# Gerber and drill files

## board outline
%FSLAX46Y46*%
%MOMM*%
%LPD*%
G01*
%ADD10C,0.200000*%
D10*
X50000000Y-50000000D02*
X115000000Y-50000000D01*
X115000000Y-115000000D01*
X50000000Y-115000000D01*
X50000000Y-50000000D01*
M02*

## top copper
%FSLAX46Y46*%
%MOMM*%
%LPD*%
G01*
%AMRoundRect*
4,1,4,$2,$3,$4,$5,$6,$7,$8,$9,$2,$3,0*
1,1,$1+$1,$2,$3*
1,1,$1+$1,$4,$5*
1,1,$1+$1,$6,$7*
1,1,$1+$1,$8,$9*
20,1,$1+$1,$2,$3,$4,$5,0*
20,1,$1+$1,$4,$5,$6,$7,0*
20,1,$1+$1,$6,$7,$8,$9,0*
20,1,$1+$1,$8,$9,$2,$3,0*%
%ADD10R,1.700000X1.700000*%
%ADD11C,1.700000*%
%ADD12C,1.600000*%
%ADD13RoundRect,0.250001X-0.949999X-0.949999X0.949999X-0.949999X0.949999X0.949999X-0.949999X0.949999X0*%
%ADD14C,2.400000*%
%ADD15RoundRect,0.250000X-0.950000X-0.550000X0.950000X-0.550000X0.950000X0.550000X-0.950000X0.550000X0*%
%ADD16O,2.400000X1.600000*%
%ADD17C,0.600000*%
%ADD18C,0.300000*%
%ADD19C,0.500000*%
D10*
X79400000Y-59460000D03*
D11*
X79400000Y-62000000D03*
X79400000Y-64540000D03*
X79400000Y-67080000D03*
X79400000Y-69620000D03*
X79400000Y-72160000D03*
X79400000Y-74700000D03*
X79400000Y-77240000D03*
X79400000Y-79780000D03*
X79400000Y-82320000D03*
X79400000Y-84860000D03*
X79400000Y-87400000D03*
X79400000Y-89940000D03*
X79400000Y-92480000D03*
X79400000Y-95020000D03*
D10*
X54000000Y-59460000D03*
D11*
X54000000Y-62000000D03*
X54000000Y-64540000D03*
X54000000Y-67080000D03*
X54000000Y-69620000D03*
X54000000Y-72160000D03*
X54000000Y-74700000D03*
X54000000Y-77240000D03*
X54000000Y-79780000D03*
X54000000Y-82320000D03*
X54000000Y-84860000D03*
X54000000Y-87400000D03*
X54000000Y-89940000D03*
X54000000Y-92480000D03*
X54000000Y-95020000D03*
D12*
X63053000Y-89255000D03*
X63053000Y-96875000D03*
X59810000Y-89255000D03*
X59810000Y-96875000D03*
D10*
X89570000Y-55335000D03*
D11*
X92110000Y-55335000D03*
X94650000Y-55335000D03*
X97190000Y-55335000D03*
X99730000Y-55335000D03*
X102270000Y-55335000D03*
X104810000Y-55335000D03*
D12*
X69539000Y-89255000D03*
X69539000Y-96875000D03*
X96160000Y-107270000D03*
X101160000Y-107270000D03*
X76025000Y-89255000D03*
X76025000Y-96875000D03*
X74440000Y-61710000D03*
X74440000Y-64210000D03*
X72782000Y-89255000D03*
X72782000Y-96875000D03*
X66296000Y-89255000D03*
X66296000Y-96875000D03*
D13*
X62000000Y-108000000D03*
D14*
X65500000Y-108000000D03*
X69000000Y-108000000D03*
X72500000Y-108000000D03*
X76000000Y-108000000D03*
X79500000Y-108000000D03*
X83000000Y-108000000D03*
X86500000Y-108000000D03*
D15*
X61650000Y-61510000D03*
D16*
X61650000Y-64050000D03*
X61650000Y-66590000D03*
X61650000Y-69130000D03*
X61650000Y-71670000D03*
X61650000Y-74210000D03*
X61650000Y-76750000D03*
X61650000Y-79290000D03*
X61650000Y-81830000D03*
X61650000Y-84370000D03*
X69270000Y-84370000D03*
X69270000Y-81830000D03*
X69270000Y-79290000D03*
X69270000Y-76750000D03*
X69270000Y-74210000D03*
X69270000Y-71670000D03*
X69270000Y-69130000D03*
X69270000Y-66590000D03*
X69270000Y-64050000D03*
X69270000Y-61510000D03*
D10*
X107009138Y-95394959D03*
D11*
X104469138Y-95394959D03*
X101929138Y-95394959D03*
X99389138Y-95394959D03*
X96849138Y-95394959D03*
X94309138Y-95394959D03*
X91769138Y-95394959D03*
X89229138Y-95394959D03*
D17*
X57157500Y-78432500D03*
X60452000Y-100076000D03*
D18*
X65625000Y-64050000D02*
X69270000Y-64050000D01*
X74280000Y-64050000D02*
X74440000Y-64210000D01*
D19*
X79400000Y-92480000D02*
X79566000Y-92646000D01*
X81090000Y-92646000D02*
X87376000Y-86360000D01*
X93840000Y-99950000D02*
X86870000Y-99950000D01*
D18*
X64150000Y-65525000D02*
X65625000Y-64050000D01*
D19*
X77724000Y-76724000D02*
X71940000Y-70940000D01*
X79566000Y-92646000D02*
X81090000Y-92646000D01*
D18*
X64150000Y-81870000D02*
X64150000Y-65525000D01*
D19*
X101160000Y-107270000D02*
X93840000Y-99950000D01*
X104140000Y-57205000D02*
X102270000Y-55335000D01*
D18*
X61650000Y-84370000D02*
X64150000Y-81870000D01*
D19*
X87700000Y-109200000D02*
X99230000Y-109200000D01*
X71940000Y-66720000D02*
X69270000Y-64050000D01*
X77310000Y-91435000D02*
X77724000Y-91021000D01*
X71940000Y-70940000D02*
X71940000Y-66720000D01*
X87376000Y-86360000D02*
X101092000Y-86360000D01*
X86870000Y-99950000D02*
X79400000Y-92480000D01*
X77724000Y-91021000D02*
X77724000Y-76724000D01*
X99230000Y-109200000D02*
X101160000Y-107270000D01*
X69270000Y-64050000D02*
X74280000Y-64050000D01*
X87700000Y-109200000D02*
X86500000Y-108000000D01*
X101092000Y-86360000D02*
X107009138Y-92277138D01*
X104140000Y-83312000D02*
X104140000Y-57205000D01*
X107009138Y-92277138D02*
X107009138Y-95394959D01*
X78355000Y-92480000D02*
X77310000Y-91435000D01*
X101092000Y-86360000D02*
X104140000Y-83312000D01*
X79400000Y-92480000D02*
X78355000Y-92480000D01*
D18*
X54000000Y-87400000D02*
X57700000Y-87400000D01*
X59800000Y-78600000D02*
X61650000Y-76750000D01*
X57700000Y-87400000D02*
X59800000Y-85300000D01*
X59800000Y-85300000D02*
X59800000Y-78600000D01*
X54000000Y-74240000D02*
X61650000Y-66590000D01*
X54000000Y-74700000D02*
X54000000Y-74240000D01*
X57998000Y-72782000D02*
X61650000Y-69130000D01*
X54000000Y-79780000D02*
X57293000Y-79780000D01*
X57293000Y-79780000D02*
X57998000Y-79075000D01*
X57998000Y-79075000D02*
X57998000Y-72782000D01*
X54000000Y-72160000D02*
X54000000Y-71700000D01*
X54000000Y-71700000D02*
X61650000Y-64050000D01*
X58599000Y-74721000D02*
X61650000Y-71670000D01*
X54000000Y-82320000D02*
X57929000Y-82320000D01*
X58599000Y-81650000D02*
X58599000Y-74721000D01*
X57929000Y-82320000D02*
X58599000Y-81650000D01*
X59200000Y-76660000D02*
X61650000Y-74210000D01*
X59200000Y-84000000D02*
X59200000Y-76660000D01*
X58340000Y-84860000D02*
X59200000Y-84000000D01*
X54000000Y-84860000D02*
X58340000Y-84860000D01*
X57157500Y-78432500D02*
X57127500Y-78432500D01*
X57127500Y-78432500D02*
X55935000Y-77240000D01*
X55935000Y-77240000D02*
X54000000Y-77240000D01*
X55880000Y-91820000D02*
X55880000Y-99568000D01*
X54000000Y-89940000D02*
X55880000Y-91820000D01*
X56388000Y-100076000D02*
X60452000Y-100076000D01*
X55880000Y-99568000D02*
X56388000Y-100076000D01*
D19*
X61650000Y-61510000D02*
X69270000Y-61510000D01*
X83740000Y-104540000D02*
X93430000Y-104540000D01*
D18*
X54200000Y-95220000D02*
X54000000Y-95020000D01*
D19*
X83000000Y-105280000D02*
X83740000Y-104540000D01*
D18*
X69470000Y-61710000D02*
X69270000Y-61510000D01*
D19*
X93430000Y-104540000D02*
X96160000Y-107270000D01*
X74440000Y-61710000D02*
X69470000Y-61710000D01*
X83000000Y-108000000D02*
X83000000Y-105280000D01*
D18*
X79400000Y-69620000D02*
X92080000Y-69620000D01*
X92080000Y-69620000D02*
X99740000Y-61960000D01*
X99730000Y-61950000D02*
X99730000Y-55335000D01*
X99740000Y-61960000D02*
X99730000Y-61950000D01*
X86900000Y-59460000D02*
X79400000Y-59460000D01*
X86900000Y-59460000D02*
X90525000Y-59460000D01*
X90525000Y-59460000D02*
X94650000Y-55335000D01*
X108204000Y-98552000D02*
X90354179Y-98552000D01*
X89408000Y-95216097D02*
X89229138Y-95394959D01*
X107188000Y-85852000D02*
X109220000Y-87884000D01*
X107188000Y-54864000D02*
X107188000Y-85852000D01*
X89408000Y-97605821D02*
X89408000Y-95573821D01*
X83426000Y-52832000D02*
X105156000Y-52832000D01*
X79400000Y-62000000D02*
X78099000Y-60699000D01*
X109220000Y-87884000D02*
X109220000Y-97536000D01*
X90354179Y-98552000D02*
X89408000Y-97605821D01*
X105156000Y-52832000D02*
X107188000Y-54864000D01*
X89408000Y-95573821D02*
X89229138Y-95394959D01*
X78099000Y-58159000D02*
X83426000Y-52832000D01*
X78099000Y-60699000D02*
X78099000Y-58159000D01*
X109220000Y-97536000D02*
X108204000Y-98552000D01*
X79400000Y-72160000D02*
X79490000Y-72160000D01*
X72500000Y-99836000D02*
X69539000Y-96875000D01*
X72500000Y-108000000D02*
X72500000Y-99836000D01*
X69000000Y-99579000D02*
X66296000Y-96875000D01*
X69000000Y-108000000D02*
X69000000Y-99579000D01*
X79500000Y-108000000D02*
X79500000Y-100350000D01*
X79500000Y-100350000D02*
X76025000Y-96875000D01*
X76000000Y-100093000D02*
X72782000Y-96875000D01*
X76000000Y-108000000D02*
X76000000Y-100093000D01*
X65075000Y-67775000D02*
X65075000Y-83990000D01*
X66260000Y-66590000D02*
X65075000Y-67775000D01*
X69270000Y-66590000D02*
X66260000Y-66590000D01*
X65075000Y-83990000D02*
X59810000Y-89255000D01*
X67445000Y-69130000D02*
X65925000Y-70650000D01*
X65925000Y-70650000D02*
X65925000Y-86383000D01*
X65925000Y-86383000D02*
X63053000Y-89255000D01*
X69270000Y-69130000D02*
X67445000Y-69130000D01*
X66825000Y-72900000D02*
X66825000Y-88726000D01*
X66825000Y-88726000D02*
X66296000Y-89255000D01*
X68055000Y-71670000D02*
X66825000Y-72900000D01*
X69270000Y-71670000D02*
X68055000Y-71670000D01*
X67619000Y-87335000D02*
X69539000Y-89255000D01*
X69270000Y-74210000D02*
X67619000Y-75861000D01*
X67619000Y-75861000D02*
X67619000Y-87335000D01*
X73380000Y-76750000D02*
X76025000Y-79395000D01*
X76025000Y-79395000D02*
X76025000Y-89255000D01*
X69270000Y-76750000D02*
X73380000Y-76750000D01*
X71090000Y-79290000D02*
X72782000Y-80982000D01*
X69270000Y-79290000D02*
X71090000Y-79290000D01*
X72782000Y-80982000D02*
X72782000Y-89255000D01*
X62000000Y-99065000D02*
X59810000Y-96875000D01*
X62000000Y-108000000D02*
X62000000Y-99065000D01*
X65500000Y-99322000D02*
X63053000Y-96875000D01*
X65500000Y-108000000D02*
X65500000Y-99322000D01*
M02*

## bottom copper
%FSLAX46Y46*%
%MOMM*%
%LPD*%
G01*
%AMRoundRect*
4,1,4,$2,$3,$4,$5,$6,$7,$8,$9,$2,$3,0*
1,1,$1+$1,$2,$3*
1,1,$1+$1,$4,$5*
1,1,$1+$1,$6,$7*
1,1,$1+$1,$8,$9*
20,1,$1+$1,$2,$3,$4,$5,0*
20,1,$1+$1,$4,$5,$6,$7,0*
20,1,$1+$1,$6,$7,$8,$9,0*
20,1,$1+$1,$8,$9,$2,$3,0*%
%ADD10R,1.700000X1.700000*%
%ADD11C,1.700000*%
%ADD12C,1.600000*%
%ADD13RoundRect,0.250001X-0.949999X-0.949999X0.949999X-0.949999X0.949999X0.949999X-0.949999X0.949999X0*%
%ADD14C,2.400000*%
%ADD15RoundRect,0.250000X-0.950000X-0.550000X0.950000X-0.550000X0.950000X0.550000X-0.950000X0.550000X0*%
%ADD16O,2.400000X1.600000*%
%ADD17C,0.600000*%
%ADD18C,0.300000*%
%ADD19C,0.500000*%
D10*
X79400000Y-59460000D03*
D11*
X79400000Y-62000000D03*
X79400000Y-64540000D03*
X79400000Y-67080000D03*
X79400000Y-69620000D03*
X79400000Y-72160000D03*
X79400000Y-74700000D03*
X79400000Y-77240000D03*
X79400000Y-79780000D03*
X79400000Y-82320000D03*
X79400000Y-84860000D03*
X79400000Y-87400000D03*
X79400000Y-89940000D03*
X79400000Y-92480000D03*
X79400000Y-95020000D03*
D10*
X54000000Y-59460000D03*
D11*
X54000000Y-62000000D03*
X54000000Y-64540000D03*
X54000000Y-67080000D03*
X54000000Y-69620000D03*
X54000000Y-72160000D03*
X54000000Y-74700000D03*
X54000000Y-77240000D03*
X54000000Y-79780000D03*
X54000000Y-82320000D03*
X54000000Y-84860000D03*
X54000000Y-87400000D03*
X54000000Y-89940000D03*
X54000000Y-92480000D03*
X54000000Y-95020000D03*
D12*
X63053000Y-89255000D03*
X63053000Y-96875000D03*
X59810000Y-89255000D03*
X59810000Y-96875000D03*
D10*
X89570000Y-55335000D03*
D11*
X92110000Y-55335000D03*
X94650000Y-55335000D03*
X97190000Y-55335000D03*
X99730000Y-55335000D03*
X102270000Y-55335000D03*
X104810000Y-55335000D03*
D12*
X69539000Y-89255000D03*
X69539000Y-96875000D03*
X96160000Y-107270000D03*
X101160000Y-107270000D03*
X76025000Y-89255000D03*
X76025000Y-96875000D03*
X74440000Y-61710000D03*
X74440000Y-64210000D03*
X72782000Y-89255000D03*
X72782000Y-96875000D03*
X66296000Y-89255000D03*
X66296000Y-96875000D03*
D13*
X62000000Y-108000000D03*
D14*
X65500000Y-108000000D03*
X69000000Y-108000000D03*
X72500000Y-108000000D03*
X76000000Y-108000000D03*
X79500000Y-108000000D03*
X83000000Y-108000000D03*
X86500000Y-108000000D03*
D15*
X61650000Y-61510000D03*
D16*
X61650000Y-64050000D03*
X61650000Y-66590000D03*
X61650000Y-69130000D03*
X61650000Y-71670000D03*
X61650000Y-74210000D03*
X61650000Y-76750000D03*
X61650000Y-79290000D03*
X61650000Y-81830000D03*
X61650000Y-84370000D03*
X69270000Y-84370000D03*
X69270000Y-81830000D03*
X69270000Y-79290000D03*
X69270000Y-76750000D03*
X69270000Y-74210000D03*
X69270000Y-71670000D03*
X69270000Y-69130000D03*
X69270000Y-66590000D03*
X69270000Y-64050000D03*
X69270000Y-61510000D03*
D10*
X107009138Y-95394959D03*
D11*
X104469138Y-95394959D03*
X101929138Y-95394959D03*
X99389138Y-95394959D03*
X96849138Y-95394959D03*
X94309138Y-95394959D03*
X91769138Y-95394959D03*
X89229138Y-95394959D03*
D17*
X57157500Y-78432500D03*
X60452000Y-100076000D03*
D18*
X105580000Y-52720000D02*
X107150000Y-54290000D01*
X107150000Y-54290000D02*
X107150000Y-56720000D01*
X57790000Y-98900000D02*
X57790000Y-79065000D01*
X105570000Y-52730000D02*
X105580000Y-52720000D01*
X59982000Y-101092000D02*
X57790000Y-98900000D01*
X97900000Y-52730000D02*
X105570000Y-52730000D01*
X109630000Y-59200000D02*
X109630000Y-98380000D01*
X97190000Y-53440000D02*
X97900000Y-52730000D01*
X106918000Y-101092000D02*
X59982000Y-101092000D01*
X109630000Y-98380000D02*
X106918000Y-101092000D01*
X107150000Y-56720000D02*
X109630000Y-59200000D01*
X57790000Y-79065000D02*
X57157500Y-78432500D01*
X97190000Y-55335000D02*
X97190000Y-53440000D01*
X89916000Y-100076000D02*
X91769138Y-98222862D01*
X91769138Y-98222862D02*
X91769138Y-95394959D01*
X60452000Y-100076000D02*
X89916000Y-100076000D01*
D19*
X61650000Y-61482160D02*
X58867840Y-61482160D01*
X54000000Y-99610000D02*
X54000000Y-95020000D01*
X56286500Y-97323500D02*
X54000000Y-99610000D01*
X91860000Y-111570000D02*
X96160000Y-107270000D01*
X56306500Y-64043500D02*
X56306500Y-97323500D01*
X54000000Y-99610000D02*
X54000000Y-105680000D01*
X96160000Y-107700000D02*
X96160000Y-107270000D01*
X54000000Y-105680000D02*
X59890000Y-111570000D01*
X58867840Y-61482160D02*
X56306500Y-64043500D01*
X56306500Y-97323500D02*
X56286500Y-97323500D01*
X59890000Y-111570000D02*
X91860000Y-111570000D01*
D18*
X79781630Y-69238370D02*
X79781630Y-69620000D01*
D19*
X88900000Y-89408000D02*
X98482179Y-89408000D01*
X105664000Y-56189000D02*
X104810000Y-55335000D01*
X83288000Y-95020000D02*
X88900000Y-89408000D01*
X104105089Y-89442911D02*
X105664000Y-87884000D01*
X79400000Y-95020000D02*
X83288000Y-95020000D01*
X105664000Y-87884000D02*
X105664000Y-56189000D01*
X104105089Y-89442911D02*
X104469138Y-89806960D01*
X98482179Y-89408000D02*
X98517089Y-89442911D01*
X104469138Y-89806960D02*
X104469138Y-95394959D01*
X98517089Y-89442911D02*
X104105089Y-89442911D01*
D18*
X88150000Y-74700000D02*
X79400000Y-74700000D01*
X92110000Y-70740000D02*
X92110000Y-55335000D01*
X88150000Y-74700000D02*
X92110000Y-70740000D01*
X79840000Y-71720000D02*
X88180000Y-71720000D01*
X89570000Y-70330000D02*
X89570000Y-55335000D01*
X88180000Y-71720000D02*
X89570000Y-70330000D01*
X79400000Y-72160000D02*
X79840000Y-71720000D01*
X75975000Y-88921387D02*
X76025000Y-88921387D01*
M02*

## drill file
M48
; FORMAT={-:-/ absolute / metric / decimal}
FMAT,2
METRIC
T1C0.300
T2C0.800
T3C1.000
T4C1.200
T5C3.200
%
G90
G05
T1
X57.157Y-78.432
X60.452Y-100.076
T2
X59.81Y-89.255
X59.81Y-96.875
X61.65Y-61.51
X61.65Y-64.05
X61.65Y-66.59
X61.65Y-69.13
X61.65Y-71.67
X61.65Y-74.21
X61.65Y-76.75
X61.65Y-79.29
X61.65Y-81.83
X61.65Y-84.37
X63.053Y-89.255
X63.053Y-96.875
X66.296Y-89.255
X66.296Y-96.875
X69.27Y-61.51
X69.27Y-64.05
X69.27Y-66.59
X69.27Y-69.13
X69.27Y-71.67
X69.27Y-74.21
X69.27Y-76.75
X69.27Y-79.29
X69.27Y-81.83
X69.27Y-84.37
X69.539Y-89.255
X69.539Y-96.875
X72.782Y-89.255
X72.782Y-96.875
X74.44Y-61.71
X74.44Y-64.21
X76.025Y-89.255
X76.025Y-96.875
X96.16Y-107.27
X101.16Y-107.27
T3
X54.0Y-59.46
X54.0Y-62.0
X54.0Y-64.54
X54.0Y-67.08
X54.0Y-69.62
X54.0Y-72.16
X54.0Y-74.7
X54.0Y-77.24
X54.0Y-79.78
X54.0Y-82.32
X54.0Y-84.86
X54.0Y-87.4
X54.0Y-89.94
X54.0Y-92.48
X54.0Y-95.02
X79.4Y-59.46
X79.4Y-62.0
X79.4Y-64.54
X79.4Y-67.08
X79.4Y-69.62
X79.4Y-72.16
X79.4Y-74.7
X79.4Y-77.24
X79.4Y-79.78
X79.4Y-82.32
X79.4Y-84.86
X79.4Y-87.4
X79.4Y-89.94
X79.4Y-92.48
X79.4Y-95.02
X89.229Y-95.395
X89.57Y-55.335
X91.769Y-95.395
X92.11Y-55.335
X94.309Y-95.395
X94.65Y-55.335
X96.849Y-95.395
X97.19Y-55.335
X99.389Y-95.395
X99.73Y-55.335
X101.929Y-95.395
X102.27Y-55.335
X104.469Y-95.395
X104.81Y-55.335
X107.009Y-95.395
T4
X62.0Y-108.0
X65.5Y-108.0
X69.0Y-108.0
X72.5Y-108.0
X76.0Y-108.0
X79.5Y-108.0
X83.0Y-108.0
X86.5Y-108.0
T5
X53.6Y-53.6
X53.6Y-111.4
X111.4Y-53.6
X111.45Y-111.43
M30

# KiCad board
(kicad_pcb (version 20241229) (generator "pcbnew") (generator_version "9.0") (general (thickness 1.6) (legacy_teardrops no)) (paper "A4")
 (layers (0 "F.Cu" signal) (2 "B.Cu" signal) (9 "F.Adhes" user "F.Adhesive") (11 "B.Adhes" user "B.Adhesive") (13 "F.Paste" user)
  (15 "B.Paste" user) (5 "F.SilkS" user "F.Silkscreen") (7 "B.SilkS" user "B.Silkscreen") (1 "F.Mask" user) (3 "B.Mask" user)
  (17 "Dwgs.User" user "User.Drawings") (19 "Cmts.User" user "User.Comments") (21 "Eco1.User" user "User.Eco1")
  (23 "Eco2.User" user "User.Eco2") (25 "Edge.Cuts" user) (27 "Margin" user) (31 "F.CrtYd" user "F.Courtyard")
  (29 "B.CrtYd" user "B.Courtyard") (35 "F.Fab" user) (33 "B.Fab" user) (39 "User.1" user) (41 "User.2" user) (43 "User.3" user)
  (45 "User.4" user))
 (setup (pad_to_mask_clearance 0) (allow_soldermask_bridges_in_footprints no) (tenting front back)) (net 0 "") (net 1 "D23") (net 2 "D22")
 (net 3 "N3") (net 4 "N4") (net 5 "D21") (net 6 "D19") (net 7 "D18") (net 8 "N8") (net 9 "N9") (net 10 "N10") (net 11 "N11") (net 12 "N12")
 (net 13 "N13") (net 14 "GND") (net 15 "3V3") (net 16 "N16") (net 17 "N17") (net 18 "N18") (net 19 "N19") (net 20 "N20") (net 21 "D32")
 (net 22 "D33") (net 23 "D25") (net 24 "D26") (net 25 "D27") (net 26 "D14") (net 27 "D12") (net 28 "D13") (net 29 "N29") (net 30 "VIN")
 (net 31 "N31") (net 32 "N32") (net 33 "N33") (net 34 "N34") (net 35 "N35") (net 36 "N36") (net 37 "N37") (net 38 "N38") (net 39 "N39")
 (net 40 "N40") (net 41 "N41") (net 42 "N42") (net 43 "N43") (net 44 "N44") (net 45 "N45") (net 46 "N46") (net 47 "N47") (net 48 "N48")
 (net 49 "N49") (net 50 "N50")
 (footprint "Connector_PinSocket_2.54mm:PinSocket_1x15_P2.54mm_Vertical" (layer "F.Cu") (at 79.4 59.46)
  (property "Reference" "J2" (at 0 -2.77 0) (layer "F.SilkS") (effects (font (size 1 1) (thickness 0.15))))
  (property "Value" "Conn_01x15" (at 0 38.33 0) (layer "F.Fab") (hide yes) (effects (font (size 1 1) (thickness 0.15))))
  (pad "1" thru_hole rect (at 0 0) (size 1.7 1.7) (drill 1) (layers "*.Cu" "*.Mask") (remove_unused_layers no) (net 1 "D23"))
  (pad "2" thru_hole circle (at 0 2.54) (size 1.7 1.7) (drill 1) (layers "*.Cu" "*.Mask") (remove_unused_layers no) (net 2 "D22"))
  (pad "3" thru_hole circle (at 0 5.08) (size 1.7 1.7) (drill 1) (layers "*.Cu" "*.Mask") (remove_unused_layers no) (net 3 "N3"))
  (pad "4" thru_hole circle (at 0 7.62) (size 1.7 1.7) (drill 1) (layers "*.Cu" "*.Mask") (remove_unused_layers no) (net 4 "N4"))
  (pad "5" thru_hole circle (at 0 10.16) (size 1.7 1.7) (drill 1) (layers "*.Cu" "*.Mask") (remove_unused_layers no) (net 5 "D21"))
  (pad "6" thru_hole circle (at 0 12.7) (size 1.7 1.7) (drill 1) (layers "*.Cu" "*.Mask") (remove_unused_layers no) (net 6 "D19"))
  (pad "7" thru_hole circle (at 0 15.24) (size 1.7 1.7) (drill 1) (layers "*.Cu" "*.Mask") (remove_unused_layers no) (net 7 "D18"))
  (pad "8" thru_hole circle (at 0 17.78) (size 1.7 1.7) (drill 1) (layers "*.Cu" "*.Mask") (remove_unused_layers no) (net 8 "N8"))
  (pad "9" thru_hole circle (at 0 20.32) (size 1.7 1.7) (drill 1) (layers "*.Cu" "*.Mask") (remove_unused_layers no) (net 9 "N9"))
  (pad "10" thru_hole circle (at 0 22.86) (size 1.7 1.7) (drill 1) (layers "*.Cu" "*.Mask") (remove_unused_layers no) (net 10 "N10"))
  (pad "11" thru_hole circle (at 0 25.4) (size 1.7 1.7) (drill 1) (layers "*.Cu" "*.Mask") (remove_unused_layers no) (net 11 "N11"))
  (pad "12" thru_hole circle (at 0 27.94) (size 1.7 1.7) (drill 1) (layers "*.Cu" "*.Mask") (remove_unused_layers no) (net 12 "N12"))
  (pad "13" thru_hole circle (at 0 30.48) (size 1.7 1.7) (drill 1) (layers "*.Cu" "*.Mask") (remove_unused_layers no) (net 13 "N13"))
  (pad "14" thru_hole circle (at 0 33.02) (size 1.7 1.7) (drill 1) (layers "*.Cu" "*.Mask") (remove_unused_layers no) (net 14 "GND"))
  (pad "15" thru_hole circle (at 0 35.56) (size 1.7 1.7) (drill 1) (layers "*.Cu" "*.Mask") (remove_unused_layers no) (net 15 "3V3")))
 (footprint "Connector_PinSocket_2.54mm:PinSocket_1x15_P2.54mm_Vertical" (layer "F.Cu") (at 54 59.46)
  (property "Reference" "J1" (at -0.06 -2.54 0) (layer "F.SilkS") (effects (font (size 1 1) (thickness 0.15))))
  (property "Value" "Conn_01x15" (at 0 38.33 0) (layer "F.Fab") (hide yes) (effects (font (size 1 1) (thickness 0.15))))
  (pad "1" thru_hole rect (at 0 0) (size 1.7 1.7) (drill 1) (layers "*.Cu" "*.Mask") (remove_unused_layers no) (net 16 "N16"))
  (pad "2" thru_hole circle (at 0 2.54) (size 1.7 1.7) (drill 1) (layers "*.Cu" "*.Mask") (remove_unused_layers no) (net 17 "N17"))
  (pad "3" thru_hole circle (at 0 5.08) (size 1.7 1.7) (drill 1) (layers "*.Cu" "*.Mask") (remove_unused_layers no) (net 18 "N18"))
  (pad "4" thru_hole circle (at 0 7.62) (size 1.7 1.7) (drill 1) (layers "*.Cu" "*.Mask") (remove_unused_layers no) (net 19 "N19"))
  (pad "5" thru_hole circle (at 0 10.16) (size 1.7 1.7) (drill 1) (layers "*.Cu" "*.Mask") (remove_unused_layers no) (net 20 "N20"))
  (pad "6" thru_hole circle (at 0 12.7) (size 1.7 1.7) (drill 1) (layers "*.Cu" "*.Mask") (remove_unused_layers no) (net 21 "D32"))
  (pad "7" thru_hole circle (at 0 15.24) (size 1.7 1.7) (drill 1) (layers "*.Cu" "*.Mask") (remove_unused_layers no) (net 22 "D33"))
  (pad "8" thru_hole circle (at 0 17.78) (size 1.7 1.7) (drill 1) (layers "*.Cu" "*.Mask") (remove_unused_layers no) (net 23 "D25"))
  (pad "9" thru_hole circle (at 0 20.32) (size 1.7 1.7) (drill 1) (layers "*.Cu" "*.Mask") (remove_unused_layers no) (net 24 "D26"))
  (pad "10" thru_hole circle (at 0 22.86) (size 1.7 1.7) (drill 1) (layers "*.Cu" "*.Mask") (remove_unused_layers no) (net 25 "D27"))
  (pad "11" thru_hole circle (at 0 25.4) (size 1.7 1.7) (drill 1) (layers "*.Cu" "*.Mask") (remove_unused_layers no) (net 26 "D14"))
  (pad "12" thru_hole circle (at 0 27.94) (size 1.7 1.7) (drill 1) (layers "*.Cu" "*.Mask") (remove_unused_layers no) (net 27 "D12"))
  (pad "13" thru_hole circle (at 0 30.48) (size 1.7 1.7) (drill 1) (layers "*.Cu" "*.Mask") (remove_unused_layers no) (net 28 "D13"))
  (pad "14" thru_hole circle (at 0 33.02) (size 1.7 1.7) (drill 1) (layers "*.Cu" "*.Mask") (remove_unused_layers no) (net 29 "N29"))
  (pad "15" thru_hole circle (at 0 35.56) (size 1.7 1.7) (drill 1) (layers "*.Cu" "*.Mask") (remove_unused_layers no) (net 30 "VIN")))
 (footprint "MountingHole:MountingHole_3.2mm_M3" (layer "F.Cu") (at 53.6 53.6)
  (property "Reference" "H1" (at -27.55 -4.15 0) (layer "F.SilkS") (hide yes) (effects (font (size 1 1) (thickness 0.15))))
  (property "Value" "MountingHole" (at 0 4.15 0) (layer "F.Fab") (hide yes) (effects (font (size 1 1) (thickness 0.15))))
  (pad "" np_thru_hole circle (at 0 0) (size 3.2 3.2) (drill 3.2) (layers "*.Cu" "*.Mask")))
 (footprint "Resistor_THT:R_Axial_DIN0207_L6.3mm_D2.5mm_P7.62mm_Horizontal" (layer "F.Cu") (at 63.053 89.255 -90)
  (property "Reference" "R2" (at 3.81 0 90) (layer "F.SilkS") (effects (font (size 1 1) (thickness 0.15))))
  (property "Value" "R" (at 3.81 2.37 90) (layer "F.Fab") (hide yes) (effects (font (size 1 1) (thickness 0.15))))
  (pad "1" thru_hole circle (at 0 0 270) (size 1.6 1.6) (drill 0.8) (layers "*.Cu" "*.Mask") (remove_unused_layers no) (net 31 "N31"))
  (pad "2" thru_hole circle (at 7.62 0 270) (size 1.6 1.6) (drill 0.8) (layers "*.Cu" "*.Mask") (remove_unused_layers no) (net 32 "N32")))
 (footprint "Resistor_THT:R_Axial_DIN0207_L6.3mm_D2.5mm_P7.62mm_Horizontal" (layer "F.Cu") (at 59.81 89.255 -90)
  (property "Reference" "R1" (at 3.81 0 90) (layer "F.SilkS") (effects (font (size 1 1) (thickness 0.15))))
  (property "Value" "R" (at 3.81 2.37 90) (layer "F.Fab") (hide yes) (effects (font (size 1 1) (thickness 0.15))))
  (pad "1" thru_hole circle (at 0 0 270) (size 1.6 1.6) (drill 0.8) (layers "*.Cu" "*.Mask") (remove_unused_layers no) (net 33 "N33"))
  (pad "2" thru_hole circle (at 7.62 0 270) (size 1.6 1.6) (drill 0.8) (layers "*.Cu" "*.Mask") (remove_unused_layers no) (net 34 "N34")))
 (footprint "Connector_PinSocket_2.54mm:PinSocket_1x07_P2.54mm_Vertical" (layer "F.Cu") (at 89.57 55.335 90)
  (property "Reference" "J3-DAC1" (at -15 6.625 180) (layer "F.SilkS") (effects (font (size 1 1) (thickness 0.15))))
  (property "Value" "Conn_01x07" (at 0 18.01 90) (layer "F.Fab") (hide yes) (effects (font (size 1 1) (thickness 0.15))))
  (pad "1" thru_hole rect (at 0 0 90) (size 1.7 1.7) (drill 1) (layers "*.Cu" "*.Mask") (remove_unused_layers no) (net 6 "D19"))
  (pad "2" thru_hole circle (at 0 2.54 90) (size 1.7 1.7) (drill 1) (layers "*.Cu" "*.Mask") (remove_unused_layers no) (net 7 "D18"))
  (pad "3" thru_hole circle (at 0 5.08 90) (size 1.7 1.7) (drill 1) (layers "*.Cu" "*.Mask") (remove_unused_layers no) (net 1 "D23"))
  (pad "4" thru_hole circle (at 0 7.62 90) (size 1.7 1.7) (drill 1) (layers "*.Cu" "*.Mask") (remove_unused_layers no) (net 23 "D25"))
  (pad "5" thru_hole circle (at 0 10.16 90) (size 1.7 1.7) (drill 1) (layers "*.Cu" "*.Mask") (remove_unused_layers no) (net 5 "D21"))
  (pad "6" thru_hole circle (at 0 12.7 90) (size 1.7 1.7) (drill 1) (layers "*.Cu" "*.Mask") (remove_unused_layers no) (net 14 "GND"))
  (pad "7" thru_hole circle (at 0 15.24 90) (size 1.7 1.7) (drill 1) (layers "*.Cu" "*.Mask") (remove_unused_layers no) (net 15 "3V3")))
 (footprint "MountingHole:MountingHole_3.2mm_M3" (layer "F.Cu") (at 53.6 111.4)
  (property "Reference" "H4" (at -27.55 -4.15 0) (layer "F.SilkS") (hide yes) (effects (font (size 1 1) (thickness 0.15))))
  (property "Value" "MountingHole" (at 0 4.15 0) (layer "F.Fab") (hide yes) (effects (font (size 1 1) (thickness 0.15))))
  (pad "" np_thru_hole circle (at 0 0) (size 3.2 3.2) (drill 3.2) (layers "*.Cu" "*.Mask")))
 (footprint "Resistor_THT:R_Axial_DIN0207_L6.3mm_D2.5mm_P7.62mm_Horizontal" (layer "F.Cu") (at 69.539 89.255 -90)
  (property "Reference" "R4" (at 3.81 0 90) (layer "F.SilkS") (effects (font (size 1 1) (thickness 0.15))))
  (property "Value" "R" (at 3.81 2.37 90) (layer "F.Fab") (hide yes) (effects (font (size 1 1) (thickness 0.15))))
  (pad "1" thru_hole circle (at 0 0 270) (size 1.6 1.6) (drill 0.8) (layers "*.Cu" "*.Mask") (remove_unused_layers no) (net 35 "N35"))
  (pad "2" thru_hole circle (at 7.62 0 270) (size 1.6 1.6) (drill 0.8) (layers "*.Cu" "*.Mask") (remove_unused_layers no) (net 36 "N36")))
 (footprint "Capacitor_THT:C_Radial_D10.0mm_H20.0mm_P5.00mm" (layer "F.Cu") (at 96.16 107.27)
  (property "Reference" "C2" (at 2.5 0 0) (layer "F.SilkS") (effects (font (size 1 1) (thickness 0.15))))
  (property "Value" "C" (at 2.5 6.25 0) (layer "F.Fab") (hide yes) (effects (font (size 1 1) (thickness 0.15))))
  (pad "1" thru_hole circle (at 0 0) (size 1.6 1.6) (drill 0.8) (layers "*.Cu" "*.Mask") (remove_unused_layers no) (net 30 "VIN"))
  (pad "2" thru_hole circle (at 5 0) (size 1.6 1.6) (drill 0.8) (layers "*.Cu" "*.Mask") (remove_unused_layers no) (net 14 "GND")))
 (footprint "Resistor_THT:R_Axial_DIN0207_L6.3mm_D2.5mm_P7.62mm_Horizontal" (layer "F.Cu") (at 76.025 89.255 -90)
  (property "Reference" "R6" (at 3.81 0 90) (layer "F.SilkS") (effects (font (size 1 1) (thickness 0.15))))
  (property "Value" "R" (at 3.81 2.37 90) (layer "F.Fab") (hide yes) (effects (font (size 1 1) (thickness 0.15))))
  (pad "1" thru_hole circle (at 0 0 270) (size 1.6 1.6) (drill 0.8) (layers "*.Cu" "*.Mask") (remove_unused_layers no) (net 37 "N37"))
  (pad "2" thru_hole circle (at 7.62 0 270) (size 1.6 1.6) (drill 0.8) (layers "*.Cu" "*.Mask") (remove_unused_layers no) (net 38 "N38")))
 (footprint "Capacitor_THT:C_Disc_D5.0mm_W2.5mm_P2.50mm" (layer "F.Cu") (at 74.44 61.71 -90)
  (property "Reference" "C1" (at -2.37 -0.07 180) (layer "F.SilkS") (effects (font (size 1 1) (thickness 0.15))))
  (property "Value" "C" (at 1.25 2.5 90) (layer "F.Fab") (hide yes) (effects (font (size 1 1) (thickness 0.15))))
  (pad "1" thru_hole circle (at 0 0 270) (size 1.6 1.6) (drill 0.8) (layers "*.Cu" "*.Mask") (remove_unused_layers no) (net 30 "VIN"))
  (pad "2" thru_hole circle (at 2.5 0 270) (size 1.6 1.6) (drill 0.8) (layers "*.Cu" "*.Mask") (remove_unused_layers no) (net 14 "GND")))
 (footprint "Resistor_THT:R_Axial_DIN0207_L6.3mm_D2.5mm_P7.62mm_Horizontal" (layer "F.Cu") (at 72.782 89.255 -90)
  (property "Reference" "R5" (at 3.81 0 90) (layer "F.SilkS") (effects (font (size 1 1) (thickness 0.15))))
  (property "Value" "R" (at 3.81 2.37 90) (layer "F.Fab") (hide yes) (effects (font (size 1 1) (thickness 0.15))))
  (pad "1" thru_hole circle (at 0 0 270) (size 1.6 1.6) (drill 0.8) (layers "*.Cu" "*.Mask") (remove_unused_layers no) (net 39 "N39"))
  (pad "2" thru_hole circle (at 7.62 0 270) (size 1.6 1.6) (drill 0.8) (layers "*.Cu" "*.Mask") (remove_unused_layers no) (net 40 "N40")))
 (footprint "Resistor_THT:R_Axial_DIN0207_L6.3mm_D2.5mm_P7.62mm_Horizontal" (layer "F.Cu") (at 66.296 89.255 -90)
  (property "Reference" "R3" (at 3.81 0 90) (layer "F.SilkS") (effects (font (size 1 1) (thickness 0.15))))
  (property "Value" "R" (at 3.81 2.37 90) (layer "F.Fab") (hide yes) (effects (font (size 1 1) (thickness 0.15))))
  (pad "1" thru_hole circle (at 0 0 270) (size 1.6 1.6) (drill 0.8) (layers "*.Cu" "*.Mask") (remove_unused_layers no) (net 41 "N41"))
  (pad "2" thru_hole circle (at 7.62 0 270) (size 1.6 1.6) (drill 0.8) (layers "*.Cu" "*.Mask") (remove_unused_layers no) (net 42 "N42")))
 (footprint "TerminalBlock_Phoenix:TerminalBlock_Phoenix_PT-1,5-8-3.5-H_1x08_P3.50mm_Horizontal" (layer "F.Cu") (at 62 108)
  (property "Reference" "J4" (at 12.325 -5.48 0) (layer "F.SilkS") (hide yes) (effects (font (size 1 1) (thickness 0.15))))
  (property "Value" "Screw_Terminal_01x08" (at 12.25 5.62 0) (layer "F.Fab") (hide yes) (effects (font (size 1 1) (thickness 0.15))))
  (pad "1" thru_hole roundrect (at 0 0) (size 2.4 2.4) (drill 1.2) (layers "*.Cu" "*.Mask") (remove_unused_layers no)
   (roundrect_rratio 0.104167) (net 34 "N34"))
  (pad "2" thru_hole circle (at 3.5 0) (size 2.4 2.4) (drill 1.2) (layers "*.Cu" "*.Mask") (remove_unused_layers no) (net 32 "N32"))
  (pad "3" thru_hole circle (at 7 0) (size 2.4 2.4) (drill 1.2) (layers "*.Cu" "*.Mask") (remove_unused_layers no) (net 42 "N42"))
  (pad "4" thru_hole circle (at 10.5 0) (size 2.4 2.4) (drill 1.2) (layers "*.Cu" "*.Mask") (remove_unused_layers no) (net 36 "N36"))
  (pad "5" thru_hole circle (at 14 0) (size 2.4 2.4) (drill 1.2) (layers "*.Cu" "*.Mask") (remove_unused_layers no) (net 40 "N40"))
  (pad "6" thru_hole circle (at 17.5 0) (size 2.4 2.4) (drill 1.2) (layers "*.Cu" "*.Mask") (remove_unused_layers no) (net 38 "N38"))
  (pad "7" thru_hole circle (at 21 0) (size 2.4 2.4) (drill 1.2) (layers "*.Cu" "*.Mask") (remove_unused_layers no) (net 30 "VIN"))
  (pad "8" thru_hole circle (at 24.5 0) (size 2.4 2.4) (drill 1.2) (layers "*.Cu" "*.Mask") (remove_unused_layers no) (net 14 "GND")))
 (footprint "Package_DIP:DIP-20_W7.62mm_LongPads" (layer "F.Cu") (at 61.65 61.51)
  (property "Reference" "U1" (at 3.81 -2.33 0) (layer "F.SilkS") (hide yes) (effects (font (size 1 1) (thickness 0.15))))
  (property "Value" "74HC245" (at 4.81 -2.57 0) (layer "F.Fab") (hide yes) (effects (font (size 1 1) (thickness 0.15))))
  (pad "1" thru_hole roundrect (at 0 0) (size 2.4 1.6) (drill 0.8) (layers "*.Cu" "*.Mask") (remove_unused_layers no)
   (roundrect_rratio 0.15625) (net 30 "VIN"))
  (pad "2" thru_hole oval (at 0 2.54) (size 2.4 1.6) (drill 0.8) (layers "*.Cu" "*.Mask") (remove_unused_layers no) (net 21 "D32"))
  (pad "3" thru_hole oval (at 0 5.08) (size 2.4 1.6) (drill 0.8) (layers "*.Cu" "*.Mask") (remove_unused_layers no) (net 22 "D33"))
  (pad "4" thru_hole oval (at 0 7.62) (size 2.4 1.6) (drill 0.8) (layers "*.Cu" "*.Mask") (remove_unused_layers no) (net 24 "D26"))
  (pad "5" thru_hole oval (at 0 10.16) (size 2.4 1.6) (drill 0.8) (layers "*.Cu" "*.Mask") (remove_unused_layers no) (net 25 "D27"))
  (pad "6" thru_hole oval (at 0 12.7) (size 2.4 1.6) (drill 0.8) (layers "*.Cu" "*.Mask") (remove_unused_layers no) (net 26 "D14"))
  (pad "7" thru_hole oval (at 0 15.24) (size 2.4 1.6) (drill 0.8) (layers "*.Cu" "*.Mask") (remove_unused_layers no) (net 27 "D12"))
  (pad "8" thru_hole oval (at 0 17.78) (size 2.4 1.6) (drill 0.8) (layers "*.Cu" "*.Mask") (remove_unused_layers no) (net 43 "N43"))
  (pad "9" thru_hole oval (at 0 20.32) (size 2.4 1.6) (drill 0.8) (layers "*.Cu" "*.Mask") (remove_unused_layers no) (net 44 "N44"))
  (pad "10" thru_hole oval (at 0 22.86) (size 2.4 1.6) (drill 0.8) (layers "*.Cu" "*.Mask") (remove_unused_layers no) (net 14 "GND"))
  (pad "11" thru_hole oval (at 7.62 22.86) (size 2.4 1.6) (drill 0.8) (layers "*.Cu" "*.Mask") (remove_unused_layers no) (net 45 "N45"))
  (pad "12" thru_hole oval (at 7.62 20.32) (size 2.4 1.6) (drill 0.8) (layers "*.Cu" "*.Mask") (remove_unused_layers no) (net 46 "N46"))
  (pad "13" thru_hole oval (at 7.62 17.78) (size 2.4 1.6) (drill 0.8) (layers "*.Cu" "*.Mask") (remove_unused_layers no) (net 39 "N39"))
  (pad "14" thru_hole oval (at 7.62 15.24) (size 2.4 1.6) (drill 0.8) (layers "*.Cu" "*.Mask") (remove_unused_layers no) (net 37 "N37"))
  (pad "15" thru_hole oval (at 7.62 12.7) (size 2.4 1.6) (drill 0.8) (layers "*.Cu" "*.Mask") (remove_unused_layers no) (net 35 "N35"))
  (pad "16" thru_hole oval (at 7.62 10.16) (size 2.4 1.6) (drill 0.8) (layers "*.Cu" "*.Mask") (remove_unused_layers no) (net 41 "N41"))
  (pad "17" thru_hole oval (at 7.62 7.62) (size 2.4 1.6) (drill 0.8) (layers "*.Cu" "*.Mask") (remove_unused_layers no) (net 31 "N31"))
  (pad "18" thru_hole oval (at 7.62 5.08) (size 2.4 1.6) (drill 0.8) (layers "*.Cu" "*.Mask") (remove_unused_layers no) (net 33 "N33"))
  (pad "19" thru_hole oval (at 7.62 2.54) (size 2.4 1.6) (drill 0.8) (layers "*.Cu" "*.Mask") (remove_unused_layers no) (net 14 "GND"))
  (pad "20" thru_hole oval (at 7.62 0) (size 2.4 1.6) (drill 0.8) (layers "*.Cu" "*.Mask") (remove_unused_layers no) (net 30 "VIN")))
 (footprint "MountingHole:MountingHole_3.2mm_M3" (layer "F.Cu") (at 111.45 111.43)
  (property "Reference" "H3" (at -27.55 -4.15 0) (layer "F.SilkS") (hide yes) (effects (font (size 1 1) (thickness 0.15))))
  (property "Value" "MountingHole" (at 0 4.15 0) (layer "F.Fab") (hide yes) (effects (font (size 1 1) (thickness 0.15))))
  (pad "" np_thru_hole circle (at 0 0) (size 3.2 3.2) (drill 3.2) (layers "*.Cu" "*.Mask")))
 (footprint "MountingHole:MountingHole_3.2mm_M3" (layer "F.Cu") (at 111.4 53.6)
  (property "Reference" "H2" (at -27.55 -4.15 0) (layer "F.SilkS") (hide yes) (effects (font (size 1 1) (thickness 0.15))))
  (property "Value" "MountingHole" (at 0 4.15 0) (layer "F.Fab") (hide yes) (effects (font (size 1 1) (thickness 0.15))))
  (pad "" np_thru_hole circle (at 0 0) (size 3.2 3.2) (drill 3.2) (layers "*.Cu" "*.Mask")))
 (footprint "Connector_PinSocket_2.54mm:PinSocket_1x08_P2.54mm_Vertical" (layer "F.Cu") (at 107.009138 95.394959 -90)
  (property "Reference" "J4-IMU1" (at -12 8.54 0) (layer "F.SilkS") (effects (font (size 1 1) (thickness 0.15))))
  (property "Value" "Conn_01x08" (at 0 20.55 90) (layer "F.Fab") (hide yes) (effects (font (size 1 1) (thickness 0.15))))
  (pad "1" thru_hole rect (at 0 0 270) (size 1.7 1.7) (drill 1) (layers "*.Cu" "*.Mask") (remove_unused_layers no) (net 14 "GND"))
  (pad "2" thru_hole circle (at 0 2.54 270) (size 1.7 1.7) (drill 1) (layers "*.Cu" "*.Mask") (remove_unused_layers no) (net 15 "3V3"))
  (pad "3" thru_hole circle (at 0 5.08 270) (size 1.7 1.7) (drill 1) (layers "*.Cu" "*.Mask") (remove_unused_layers no) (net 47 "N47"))
  (pad "4" thru_hole circle (at 0 7.62 270) (size 1.7 1.7) (drill 1) (layers "*.Cu" "*.Mask") (remove_unused_layers no) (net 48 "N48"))
  (pad "5" thru_hole circle (at 0 10.16 270) (size 1.7 1.7) (drill 1) (layers "*.Cu" "*.Mask") (remove_unused_layers no) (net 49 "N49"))
  (pad "6" thru_hole circle (at 0 12.7 270) (size 1.7 1.7) (drill 1) (layers "*.Cu" "*.Mask") (remove_unused_layers no) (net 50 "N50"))
  (pad "7" thru_hole circle (at 0 15.24 270) (size 1.7 1.7) (drill 1) (layers "*.Cu" "*.Mask") (remove_unused_layers no) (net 28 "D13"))
  (pad "8" thru_hole circle (at 0 17.78 270) (size 1.7 1.7) (drill 1) (layers "*.Cu" "*.Mask") (remove_unused_layers no) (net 2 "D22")))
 (gr_rect (start 50 50) (end 115 115) (stroke (width 0.2) (type solid)) (fill no) (layer "Edge.Cuts"))
 (segment (start 65.625 64.05) (end 69.27 64.05) (width 0.3) (layer "F.Cu") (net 14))
 (segment (start 74.28 64.05) (end 74.44 64.21) (width 0.3) (layer "F.Cu") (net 14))
 (segment (start 79.4 92.48) (end 79.566 92.646) (width 0.5) (layer "F.Cu") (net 14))
 (segment (start 81.09 92.646) (end 87.376 86.36) (width 0.5) (layer "F.Cu") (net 14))
 (segment (start 93.84 99.95) (end 86.87 99.95) (width 0.5) (layer "F.Cu") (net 14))
 (segment (start 64.15 65.525) (end 65.625 64.05) (width 0.3) (layer "F.Cu") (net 14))
 (segment (start 77.724 76.724) (end 71.94 70.94) (width 0.5) (layer "F.Cu") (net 14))
 (segment (start 79.566 92.646) (end 81.09 92.646) (width 0.5) (layer "F.Cu") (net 14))
 (segment (start 64.15 81.87) (end 64.15 65.525) (width 0.3) (layer "F.Cu") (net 14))
 (segment (start 101.16 107.27) (end 93.84 99.95) (width 0.5) (layer "F.Cu") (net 14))
 (segment (start 104.14 57.205) (end 102.27 55.335) (width 0.5) (layer "F.Cu") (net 14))
 (segment (start 61.65 84.37) (end 64.15 81.87) (width 0.3) (layer "F.Cu") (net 14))
 (segment (start 87.7 109.2) (end 99.23 109.2) (width 0.5) (layer "F.Cu") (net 14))
 (segment (start 71.94 66.72) (end 69.27 64.05) (width 0.5) (layer "F.Cu") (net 14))
 (segment (start 77.31 91.435) (end 77.724 91.021) (width 0.5) (layer "F.Cu") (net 14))
 (segment (start 71.94 70.94) (end 71.94 66.72) (width 0.5) (layer "F.Cu") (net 14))
 (segment (start 87.376 86.36) (end 101.092 86.36) (width 0.5) (layer "F.Cu") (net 14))
 (segment (start 86.87 99.95) (end 79.4 92.48) (width 0.5) (layer "F.Cu") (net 14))
 (segment (start 77.724 91.021) (end 77.724 76.724) (width 0.5) (layer "F.Cu") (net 14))
 (segment (start 99.23 109.2) (end 101.16 107.27) (width 0.5) (layer "F.Cu") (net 14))
 (segment (start 69.27 64.05) (end 74.28 64.05) (width 0.5) (layer "F.Cu") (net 14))
 (segment (start 87.7 109.2) (end 86.5 108) (width 0.5) (layer "F.Cu") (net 14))
 (segment (start 101.092 86.36) (end 107.009138 92.277138) (width 0.5) (layer "F.Cu") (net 14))
 (segment (start 104.14 83.312) (end 104.14 57.205) (width 0.5) (layer "F.Cu") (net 14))
 (segment (start 107.009138 92.277138) (end 107.009138 95.394959) (width 0.5) (layer "F.Cu") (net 14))
 (segment (start 78.355 92.48) (end 77.31 91.435) (width 0.5) (layer "F.Cu") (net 14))
 (segment (start 101.092 86.36) (end 104.14 83.312) (width 0.5) (layer "F.Cu") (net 14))
 (segment (start 79.4 92.48) (end 78.355 92.48) (width 0.5) (layer "F.Cu") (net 14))
 (segment (start 54 87.4) (end 57.7 87.4) (width 0.3) (layer "F.Cu") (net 27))
 (segment (start 59.8 78.6) (end 61.65 76.75) (width 0.3) (layer "F.Cu") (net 27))
 (segment (start 57.7 87.4) (end 59.8 85.3) (width 0.3) (layer "F.Cu") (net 27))
 (segment (start 59.8 85.3) (end 59.8 78.6) (width 0.3) (layer "F.Cu") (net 27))
 (segment (start 54 74.24) (end 61.65 66.59) (width 0.3) (layer "F.Cu") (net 22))
 (segment (start 54 74.7) (end 54 74.24) (width 0.3) (layer "F.Cu") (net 22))
 (segment (start 57.998 72.782) (end 61.65 69.13) (width 0.3) (layer "F.Cu") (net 24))
 (segment (start 54 79.78) (end 57.293 79.78) (width 0.3) (layer "F.Cu") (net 24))
 (segment (start 57.293 79.78) (end 57.998 79.075) (width 0.3) (layer "F.Cu") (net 24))
 (segment (start 57.998 79.075) (end 57.998 72.782) (width 0.3) (layer "F.Cu") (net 24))
 (segment (start 54 72.16) (end 54 71.7) (width 0.3) (layer "F.Cu") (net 21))
 (segment (start 54 71.7) (end 61.65 64.05) (width 0.3) (layer "F.Cu") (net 21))
 (segment (start 58.599 74.721) (end 61.65 71.67) (width 0.3) (layer "F.Cu") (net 25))
 (segment (start 54 82.32) (end 57.929 82.32) (width 0.3) (layer "F.Cu") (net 25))
 (segment (start 58.599 81.65) (end 58.599 74.721) (width 0.3) (layer "F.Cu") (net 25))
 (segment (start 57.929 82.32) (end 58.599 81.65) (width 0.3) (layer "F.Cu") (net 25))
 (segment (start 59.2 76.66) (end 61.65 74.21) (width 0.3) (layer "F.Cu") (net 26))
 (segment (start 59.2 84) (end 59.2 76.66) (width 0.3) (layer "F.Cu") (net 26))
 (segment (start 58.34 84.86) (end 59.2 84) (width 0.3) (layer "F.Cu") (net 26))
 (segment (start 54 84.86) (end 58.34 84.86) (width 0.3) (layer "F.Cu") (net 26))
 (segment (start 57.1575 78.4325) (end 57.1275 78.4325) (width 0.3) (layer "F.Cu") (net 23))
 (segment (start 57.1275 78.4325) (end 55.935 77.24) (width 0.3) (layer "F.Cu") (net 23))
 (segment (start 55.935 77.24) (end 54 77.24) (width 0.3) (layer "F.Cu") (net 23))
 (via (at 57.1575 78.4325) (size 0.6) (drill 0.3) (layers "F.Cu" "B.Cu") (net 23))
 (segment (start 105.58 52.72) (end 107.15 54.29) (width 0.3) (layer "B.Cu") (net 23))
 (segment (start 107.15 54.29) (end 107.15 56.72) (width 0.3) (layer "B.Cu") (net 23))
 (segment (start 57.79 98.9) (end 57.79 79.065) (width 0.3) (layer "B.Cu") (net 23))
 (segment (start 105.57 52.73) (end 105.58 52.72) (width 0.3) (layer "B.Cu") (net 23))
 (segment (start 59.982 101.092) (end 57.79 98.9) (width 0.3) (layer "B.Cu") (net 23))
 (segment (start 97.9 52.73) (end 105.57 52.73) (width 0.3) (layer "B.Cu") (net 23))
 (segment (start 109.63 59.2) (end 109.63 98.38) (width 0.3) (layer "B.Cu") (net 23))
 (segment (start 97.19 53.44) (end 97.9 52.73) (width 0.3) (layer "B.Cu") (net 23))
 (segment (start 106.918 101.092) (end 59.982 101.092) (width 0.3) (layer "B.Cu") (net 23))
 (segment (start 109.63 98.38) (end 106.918 101.092) (width 0.3) (layer "B.Cu") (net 23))
 (segment (start 107.15 56.72) (end 109.63 59.2) (width 0.3) (layer "B.Cu") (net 23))
 (segment (start 57.79 79.065) (end 57.1575 78.4325) (width 0.3) (layer "B.Cu") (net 23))
 (segment (start 97.19 55.335) (end 97.19 53.44) (width 0.3) (layer "B.Cu") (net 23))
 (segment (start 55.88 91.82) (end 55.88 99.568) (width 0.3) (layer "F.Cu") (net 28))
 (segment (start 54 89.94) (end 55.88 91.82) (width 0.3) (layer "F.Cu") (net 28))
 (segment (start 56.388 100.076) (end 60.452 100.076) (width 0.3) (layer "F.Cu") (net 28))
 (segment (start 55.88 99.568) (end 56.388 100.076) (width 0.3) (layer "F.Cu") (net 28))
 (via (at 60.452 100.076) (size 0.6) (drill 0.3) (layers "F.Cu" "B.Cu") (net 28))
 (segment (start 89.916 100.076) (end 91.769138 98.222862) (width 0.3) (layer "B.Cu") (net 28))
 (segment (start 91.769138 98.222862) (end 91.769138 95.394959) (width 0.3) (layer "B.Cu") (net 28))
 (segment (start 60.452 100.076) (end 89.916 100.076) (width 0.3) (layer "B.Cu") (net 28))
 (segment (start 61.65 61.51) (end 69.27 61.51) (width 0.5) (layer "F.Cu") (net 30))
 (segment (start 83.74 104.54) (end 93.43 104.54) (width 0.5) (layer "F.Cu") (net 30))
 (segment (start 54.2 95.22) (end 54 95.02) (width 0.3) (layer "F.Cu") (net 30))
 (segment (start 83 105.28) (end 83.74 104.54) (width 0.5) (layer "F.Cu") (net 30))
 (segment (start 69.47 61.71) (end 69.27 61.51) (width 0.3) (layer "F.Cu") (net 30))
 (segment (start 93.43 104.54) (end 96.16 107.27) (width 0.5) (layer "F.Cu") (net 30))
 (segment (start 74.44 61.71) (end 69.47 61.71) (width 0.5) (layer "F.Cu") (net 30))
 (segment (start 83 108) (end 83 105.28) (width 0.5) (layer "F.Cu") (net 30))
 (segment (start 61.65 61.48216) (end 58.86784 61.48216) (width 0.5) (layer "B.Cu") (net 30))
 (segment (start 54 99.61) (end 54 95.02) (width 0.5) (layer "B.Cu") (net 30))
 (segment (start 56.2865 97.3235) (end 54 99.61) (width 0.5) (layer "B.Cu") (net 30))
 (segment (start 91.86 111.57) (end 96.16 107.27) (width 0.5) (layer "B.Cu") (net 30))
 (segment (start 56.3065 64.0435) (end 56.3065 97.3235) (width 0.5) (layer "B.Cu") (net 30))
 (segment (start 54 99.61) (end 54 105.68) (width 0.5) (layer "B.Cu") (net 30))
 (segment (start 96.16 107.7) (end 96.16 107.27) (width 0.5) (layer "B.Cu") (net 30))
 (segment (start 54 105.68) (end 59.89 111.57) (width 0.5) (layer "B.Cu") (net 30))
 (segment (start 58.86784 61.48216) (end 56.3065 64.0435) (width 0.5) (layer "B.Cu") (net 30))
 (segment (start 56.3065 97.3235) (end 56.2865 97.3235) (width 0.5) (layer "B.Cu") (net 30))
 (segment (start 59.89 111.57) (end 91.86 111.57) (width 0.5) (layer "B.Cu") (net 30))
 (segment (start 79.4 69.62) (end 92.08 69.62) (width 0.3) (layer "F.Cu") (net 5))
 (segment (start 92.08 69.62) (end 99.74 61.96) (width 0.3) (layer "F.Cu") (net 5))
 (segment (start 99.73 61.95) (end 99.73 55.335) (width 0.3) (layer "F.Cu") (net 5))
 (segment (start 99.74 61.96) (end 99.73 61.95) (width 0.3) (layer "F.Cu") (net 5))
 (segment (start 79.78163 69.23837) (end 79.78163 69.62) (width 0.3) (layer "B.Cu") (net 5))
 (segment (start 86.9 59.46) (end 79.4 59.46) (width 0.3) (layer "F.Cu") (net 1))
 (segment (start 86.9 59.46) (end 90.525 59.46) (width 0.3) (layer "F.Cu") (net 1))
 (segment (start 90.525 59.46) (end 94.65 55.335) (width 0.3) (layer "F.Cu") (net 1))
 (segment (start 108.204 98.552) (end 90.354179 98.552) (width 0.3) (layer "F.Cu") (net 2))
 (segment (start 89.408 95.216097) (end 89.229138 95.394959) (width 0.3) (layer "F.Cu") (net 2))
 (segment (start 107.188 85.852) (end 109.22 87.884) (width 0.3) (layer "F.Cu") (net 2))
 (segment (start 107.188 54.864) (end 107.188 85.852) (width 0.3) (layer "F.Cu") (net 2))
 (segment (start 89.408 97.605821) (end 89.408 95.573821) (width 0.3) (layer "F.Cu") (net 2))
 (segment (start 83.426 52.832) (end 105.156 52.832) (width 0.3) (layer "F.Cu") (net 2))
 (segment (start 79.4 62) (end 78.099 60.699) (width 0.3) (layer "F.Cu") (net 2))
 (segment (start 109.22 87.884) (end 109.22 97.536) (width 0.3) (layer "F.Cu") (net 2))
 (segment (start 90.354179 98.552) (end 89.408 97.605821) (width 0.3) (layer "F.Cu") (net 2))
 (segment (start 105.156 52.832) (end 107.188 54.864) (width 0.3) (layer "F.Cu") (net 2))
 (segment (start 89.408 95.573821) (end 89.229138 95.394959) (width 0.3) (layer "F.Cu") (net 2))
 (segment (start 78.099 58.159) (end 83.426 52.832) (width 0.3) (layer "F.Cu") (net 2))
 (segment (start 78.099 60.699) (end 78.099 58.159) (width 0.3) (layer "F.Cu") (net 2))
 (segment (start 109.22 97.536) (end 108.204 98.552) (width 0.3) (layer "F.Cu") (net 2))
 (segment (start 88.9 89.408) (end 98.482179 89.408) (width 0.5) (layer "B.Cu") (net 15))
 (segment (start 105.664 56.189) (end 104.81 55.335) (width 0.5) (layer "B.Cu") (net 15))
 (segment (start 83.288 95.02) (end 88.9 89.408) (width 0.5) (layer "B.Cu") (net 15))
 (segment (start 104.105089 89.442911) (end 105.664 87.884) (width 0.5) (layer "B.Cu") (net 15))
 (segment (start 79.4 95.02) (end 83.288 95.02) (width 0.5) (layer "B.Cu") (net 15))
 (segment (start 105.664 87.884) (end 105.664 56.189) (width 0.5) (layer "B.Cu") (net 15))
 (segment (start 104.105089 89.442911) (end 104.469138 89.80696) (width 0.5) (layer "B.Cu") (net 15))
 (segment (start 98.482179 89.408) (end 98.517089 89.442911) (width 0.5) (layer "B.Cu") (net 15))
 (segment (start 104.469138 89.80696) (end 104.469138 95.394959) (width 0.5) (layer "B.Cu") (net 15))
 (segment (start 98.517089 89.442911) (end 104.105089 89.442911) (width 0.5) (layer "B.Cu") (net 15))
 (segment (start 88.15 74.7) (end 79.4 74.7) (width 0.3) (layer "B.Cu") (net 7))
 (segment (start 92.11 70.74) (end 92.11 55.335) (width 0.3) (layer "B.Cu") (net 7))
 (segment (start 88.15 74.7) (end 92.11 70.74) (width 0.3) (layer "B.Cu") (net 7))
 (segment (start 79.4 72.16) (end 79.49 72.16) (width 0.3) (layer "F.Cu") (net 6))
 (segment (start 79.84 71.72) (end 88.18 71.72) (width 0.3) (layer "B.Cu") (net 6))
 (segment (start 89.57 70.33) (end 89.57 55.335) (width 0.3) (layer "B.Cu") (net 6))
 (segment (start 88.18 71.72) (end 89.57 70.33) (width 0.3) (layer "B.Cu") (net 6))
 (segment (start 79.4 72.16) (end 79.84 71.72) (width 0.3) (layer "B.Cu") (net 6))
 (segment (start 72.5 99.836) (end 69.539 96.875) (width 0.3) (layer "F.Cu") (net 36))
 (segment (start 72.5 108) (end 72.5 99.836) (width 0.3) (layer "F.Cu") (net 36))
 (segment (start 69 99.579) (end 66.296 96.875) (width 0.3) (layer "F.Cu") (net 42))
 (segment (start 69 108) (end 69 99.579) (width 0.3) (layer "F.Cu") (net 42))
 (segment (start 79.5 108) (end 79.5 100.35) (width 0.3) (layer "F.Cu") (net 38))
 (segment (start 79.5 100.35) (end 76.025 96.875) (width 0.3) (layer "F.Cu") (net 38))
 (segment (start 76 100.093) (end 72.782 96.875) (width 0.3) (layer "F.Cu") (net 40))
 (segment (start 76 108) (end 76 100.093) (width 0.3) (layer "F.Cu") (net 40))
 (segment (start 65.075 67.775) (end 65.075 83.99) (width 0.3) (layer "F.Cu") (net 33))
 (segment (start 66.26 66.59) (end 65.075 67.775) (width 0.3) (layer "F.Cu") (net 33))
 (segment (start 69.27 66.59) (end 66.26 66.59) (width 0.3) (layer "F.Cu") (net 33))
 (segment (start 65.075 83.99) (end 59.81 89.255) (width 0.3) (layer "F.Cu") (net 33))
 (segment (start 67.445 69.13) (end 65.925 70.65) (width 0.3) (layer "F.Cu") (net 31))
 (segment (start 65.925 70.65) (end 65.925 86.383) (width 0.3) (layer "F.Cu") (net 31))
 (segment (start 65.925 86.383) (end 63.053 89.255) (width 0.3) (layer "F.Cu") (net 31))
 (segment (start 69.27 69.13) (end 67.445 69.13) (width 0.3) (layer "F.Cu") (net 31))
 (segment (start 66.825 72.9) (end 66.825 88.726) (width 0.3) (layer "F.Cu") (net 41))
 (segment (start 66.825 88.726) (end 66.296 89.255) (width 0.3) (layer "F.Cu") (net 41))
 (segment (start 68.055 71.67) (end 66.825 72.9) (width 0.3) (layer "F.Cu") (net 41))
 (segment (start 69.27 71.67) (end 68.055 71.67) (width 0.3) (layer "F.Cu") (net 41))
 (segment (start 67.619 87.335) (end 69.539 89.255) (width 0.3) (layer "F.Cu") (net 35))
 (segment (start 69.27 74.21) (end 67.619 75.861) (width 0.3) (layer "F.Cu") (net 35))
 (segment (start 67.619 75.861) (end 67.619 87.335) (width 0.3) (layer "F.Cu") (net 35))
 (segment (start 73.38 76.75) (end 76.025 79.395) (width 0.3) (layer "F.Cu") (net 37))
 (segment (start 76.025 79.395) (end 76.025 89.255) (width 0.3) (layer "F.Cu") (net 37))
 (segment (start 69.27 76.75) (end 73.38 76.75) (width 0.3) (layer "F.Cu") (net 37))
 (segment (start 75.975 88.921387) (end 76.025 88.921387) (width 0.3) (layer "B.Cu") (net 37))
 (segment (start 71.09 79.29) (end 72.782 80.982) (width 0.3) (layer "F.Cu") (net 39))
 (segment (start 69.27 79.29) (end 71.09 79.29) (width 0.3) (layer "F.Cu") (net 39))
 (segment (start 72.782 80.982) (end 72.782 89.255) (width 0.3) (layer "F.Cu") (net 39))
 (segment (start 62 99.065) (end 59.81 96.875) (width 0.3) (layer "F.Cu") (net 34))
 (segment (start 62 108) (end 62 99.065) (width 0.3) (layer "F.Cu") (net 34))
 (segment (start 65.5 99.322) (end 63.053 96.875) (width 0.3) (layer "F.Cu") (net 32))
 (segment (start 65.5 108) (end 65.5 99.322) (width 0.3) (layer "F.Cu") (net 32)))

